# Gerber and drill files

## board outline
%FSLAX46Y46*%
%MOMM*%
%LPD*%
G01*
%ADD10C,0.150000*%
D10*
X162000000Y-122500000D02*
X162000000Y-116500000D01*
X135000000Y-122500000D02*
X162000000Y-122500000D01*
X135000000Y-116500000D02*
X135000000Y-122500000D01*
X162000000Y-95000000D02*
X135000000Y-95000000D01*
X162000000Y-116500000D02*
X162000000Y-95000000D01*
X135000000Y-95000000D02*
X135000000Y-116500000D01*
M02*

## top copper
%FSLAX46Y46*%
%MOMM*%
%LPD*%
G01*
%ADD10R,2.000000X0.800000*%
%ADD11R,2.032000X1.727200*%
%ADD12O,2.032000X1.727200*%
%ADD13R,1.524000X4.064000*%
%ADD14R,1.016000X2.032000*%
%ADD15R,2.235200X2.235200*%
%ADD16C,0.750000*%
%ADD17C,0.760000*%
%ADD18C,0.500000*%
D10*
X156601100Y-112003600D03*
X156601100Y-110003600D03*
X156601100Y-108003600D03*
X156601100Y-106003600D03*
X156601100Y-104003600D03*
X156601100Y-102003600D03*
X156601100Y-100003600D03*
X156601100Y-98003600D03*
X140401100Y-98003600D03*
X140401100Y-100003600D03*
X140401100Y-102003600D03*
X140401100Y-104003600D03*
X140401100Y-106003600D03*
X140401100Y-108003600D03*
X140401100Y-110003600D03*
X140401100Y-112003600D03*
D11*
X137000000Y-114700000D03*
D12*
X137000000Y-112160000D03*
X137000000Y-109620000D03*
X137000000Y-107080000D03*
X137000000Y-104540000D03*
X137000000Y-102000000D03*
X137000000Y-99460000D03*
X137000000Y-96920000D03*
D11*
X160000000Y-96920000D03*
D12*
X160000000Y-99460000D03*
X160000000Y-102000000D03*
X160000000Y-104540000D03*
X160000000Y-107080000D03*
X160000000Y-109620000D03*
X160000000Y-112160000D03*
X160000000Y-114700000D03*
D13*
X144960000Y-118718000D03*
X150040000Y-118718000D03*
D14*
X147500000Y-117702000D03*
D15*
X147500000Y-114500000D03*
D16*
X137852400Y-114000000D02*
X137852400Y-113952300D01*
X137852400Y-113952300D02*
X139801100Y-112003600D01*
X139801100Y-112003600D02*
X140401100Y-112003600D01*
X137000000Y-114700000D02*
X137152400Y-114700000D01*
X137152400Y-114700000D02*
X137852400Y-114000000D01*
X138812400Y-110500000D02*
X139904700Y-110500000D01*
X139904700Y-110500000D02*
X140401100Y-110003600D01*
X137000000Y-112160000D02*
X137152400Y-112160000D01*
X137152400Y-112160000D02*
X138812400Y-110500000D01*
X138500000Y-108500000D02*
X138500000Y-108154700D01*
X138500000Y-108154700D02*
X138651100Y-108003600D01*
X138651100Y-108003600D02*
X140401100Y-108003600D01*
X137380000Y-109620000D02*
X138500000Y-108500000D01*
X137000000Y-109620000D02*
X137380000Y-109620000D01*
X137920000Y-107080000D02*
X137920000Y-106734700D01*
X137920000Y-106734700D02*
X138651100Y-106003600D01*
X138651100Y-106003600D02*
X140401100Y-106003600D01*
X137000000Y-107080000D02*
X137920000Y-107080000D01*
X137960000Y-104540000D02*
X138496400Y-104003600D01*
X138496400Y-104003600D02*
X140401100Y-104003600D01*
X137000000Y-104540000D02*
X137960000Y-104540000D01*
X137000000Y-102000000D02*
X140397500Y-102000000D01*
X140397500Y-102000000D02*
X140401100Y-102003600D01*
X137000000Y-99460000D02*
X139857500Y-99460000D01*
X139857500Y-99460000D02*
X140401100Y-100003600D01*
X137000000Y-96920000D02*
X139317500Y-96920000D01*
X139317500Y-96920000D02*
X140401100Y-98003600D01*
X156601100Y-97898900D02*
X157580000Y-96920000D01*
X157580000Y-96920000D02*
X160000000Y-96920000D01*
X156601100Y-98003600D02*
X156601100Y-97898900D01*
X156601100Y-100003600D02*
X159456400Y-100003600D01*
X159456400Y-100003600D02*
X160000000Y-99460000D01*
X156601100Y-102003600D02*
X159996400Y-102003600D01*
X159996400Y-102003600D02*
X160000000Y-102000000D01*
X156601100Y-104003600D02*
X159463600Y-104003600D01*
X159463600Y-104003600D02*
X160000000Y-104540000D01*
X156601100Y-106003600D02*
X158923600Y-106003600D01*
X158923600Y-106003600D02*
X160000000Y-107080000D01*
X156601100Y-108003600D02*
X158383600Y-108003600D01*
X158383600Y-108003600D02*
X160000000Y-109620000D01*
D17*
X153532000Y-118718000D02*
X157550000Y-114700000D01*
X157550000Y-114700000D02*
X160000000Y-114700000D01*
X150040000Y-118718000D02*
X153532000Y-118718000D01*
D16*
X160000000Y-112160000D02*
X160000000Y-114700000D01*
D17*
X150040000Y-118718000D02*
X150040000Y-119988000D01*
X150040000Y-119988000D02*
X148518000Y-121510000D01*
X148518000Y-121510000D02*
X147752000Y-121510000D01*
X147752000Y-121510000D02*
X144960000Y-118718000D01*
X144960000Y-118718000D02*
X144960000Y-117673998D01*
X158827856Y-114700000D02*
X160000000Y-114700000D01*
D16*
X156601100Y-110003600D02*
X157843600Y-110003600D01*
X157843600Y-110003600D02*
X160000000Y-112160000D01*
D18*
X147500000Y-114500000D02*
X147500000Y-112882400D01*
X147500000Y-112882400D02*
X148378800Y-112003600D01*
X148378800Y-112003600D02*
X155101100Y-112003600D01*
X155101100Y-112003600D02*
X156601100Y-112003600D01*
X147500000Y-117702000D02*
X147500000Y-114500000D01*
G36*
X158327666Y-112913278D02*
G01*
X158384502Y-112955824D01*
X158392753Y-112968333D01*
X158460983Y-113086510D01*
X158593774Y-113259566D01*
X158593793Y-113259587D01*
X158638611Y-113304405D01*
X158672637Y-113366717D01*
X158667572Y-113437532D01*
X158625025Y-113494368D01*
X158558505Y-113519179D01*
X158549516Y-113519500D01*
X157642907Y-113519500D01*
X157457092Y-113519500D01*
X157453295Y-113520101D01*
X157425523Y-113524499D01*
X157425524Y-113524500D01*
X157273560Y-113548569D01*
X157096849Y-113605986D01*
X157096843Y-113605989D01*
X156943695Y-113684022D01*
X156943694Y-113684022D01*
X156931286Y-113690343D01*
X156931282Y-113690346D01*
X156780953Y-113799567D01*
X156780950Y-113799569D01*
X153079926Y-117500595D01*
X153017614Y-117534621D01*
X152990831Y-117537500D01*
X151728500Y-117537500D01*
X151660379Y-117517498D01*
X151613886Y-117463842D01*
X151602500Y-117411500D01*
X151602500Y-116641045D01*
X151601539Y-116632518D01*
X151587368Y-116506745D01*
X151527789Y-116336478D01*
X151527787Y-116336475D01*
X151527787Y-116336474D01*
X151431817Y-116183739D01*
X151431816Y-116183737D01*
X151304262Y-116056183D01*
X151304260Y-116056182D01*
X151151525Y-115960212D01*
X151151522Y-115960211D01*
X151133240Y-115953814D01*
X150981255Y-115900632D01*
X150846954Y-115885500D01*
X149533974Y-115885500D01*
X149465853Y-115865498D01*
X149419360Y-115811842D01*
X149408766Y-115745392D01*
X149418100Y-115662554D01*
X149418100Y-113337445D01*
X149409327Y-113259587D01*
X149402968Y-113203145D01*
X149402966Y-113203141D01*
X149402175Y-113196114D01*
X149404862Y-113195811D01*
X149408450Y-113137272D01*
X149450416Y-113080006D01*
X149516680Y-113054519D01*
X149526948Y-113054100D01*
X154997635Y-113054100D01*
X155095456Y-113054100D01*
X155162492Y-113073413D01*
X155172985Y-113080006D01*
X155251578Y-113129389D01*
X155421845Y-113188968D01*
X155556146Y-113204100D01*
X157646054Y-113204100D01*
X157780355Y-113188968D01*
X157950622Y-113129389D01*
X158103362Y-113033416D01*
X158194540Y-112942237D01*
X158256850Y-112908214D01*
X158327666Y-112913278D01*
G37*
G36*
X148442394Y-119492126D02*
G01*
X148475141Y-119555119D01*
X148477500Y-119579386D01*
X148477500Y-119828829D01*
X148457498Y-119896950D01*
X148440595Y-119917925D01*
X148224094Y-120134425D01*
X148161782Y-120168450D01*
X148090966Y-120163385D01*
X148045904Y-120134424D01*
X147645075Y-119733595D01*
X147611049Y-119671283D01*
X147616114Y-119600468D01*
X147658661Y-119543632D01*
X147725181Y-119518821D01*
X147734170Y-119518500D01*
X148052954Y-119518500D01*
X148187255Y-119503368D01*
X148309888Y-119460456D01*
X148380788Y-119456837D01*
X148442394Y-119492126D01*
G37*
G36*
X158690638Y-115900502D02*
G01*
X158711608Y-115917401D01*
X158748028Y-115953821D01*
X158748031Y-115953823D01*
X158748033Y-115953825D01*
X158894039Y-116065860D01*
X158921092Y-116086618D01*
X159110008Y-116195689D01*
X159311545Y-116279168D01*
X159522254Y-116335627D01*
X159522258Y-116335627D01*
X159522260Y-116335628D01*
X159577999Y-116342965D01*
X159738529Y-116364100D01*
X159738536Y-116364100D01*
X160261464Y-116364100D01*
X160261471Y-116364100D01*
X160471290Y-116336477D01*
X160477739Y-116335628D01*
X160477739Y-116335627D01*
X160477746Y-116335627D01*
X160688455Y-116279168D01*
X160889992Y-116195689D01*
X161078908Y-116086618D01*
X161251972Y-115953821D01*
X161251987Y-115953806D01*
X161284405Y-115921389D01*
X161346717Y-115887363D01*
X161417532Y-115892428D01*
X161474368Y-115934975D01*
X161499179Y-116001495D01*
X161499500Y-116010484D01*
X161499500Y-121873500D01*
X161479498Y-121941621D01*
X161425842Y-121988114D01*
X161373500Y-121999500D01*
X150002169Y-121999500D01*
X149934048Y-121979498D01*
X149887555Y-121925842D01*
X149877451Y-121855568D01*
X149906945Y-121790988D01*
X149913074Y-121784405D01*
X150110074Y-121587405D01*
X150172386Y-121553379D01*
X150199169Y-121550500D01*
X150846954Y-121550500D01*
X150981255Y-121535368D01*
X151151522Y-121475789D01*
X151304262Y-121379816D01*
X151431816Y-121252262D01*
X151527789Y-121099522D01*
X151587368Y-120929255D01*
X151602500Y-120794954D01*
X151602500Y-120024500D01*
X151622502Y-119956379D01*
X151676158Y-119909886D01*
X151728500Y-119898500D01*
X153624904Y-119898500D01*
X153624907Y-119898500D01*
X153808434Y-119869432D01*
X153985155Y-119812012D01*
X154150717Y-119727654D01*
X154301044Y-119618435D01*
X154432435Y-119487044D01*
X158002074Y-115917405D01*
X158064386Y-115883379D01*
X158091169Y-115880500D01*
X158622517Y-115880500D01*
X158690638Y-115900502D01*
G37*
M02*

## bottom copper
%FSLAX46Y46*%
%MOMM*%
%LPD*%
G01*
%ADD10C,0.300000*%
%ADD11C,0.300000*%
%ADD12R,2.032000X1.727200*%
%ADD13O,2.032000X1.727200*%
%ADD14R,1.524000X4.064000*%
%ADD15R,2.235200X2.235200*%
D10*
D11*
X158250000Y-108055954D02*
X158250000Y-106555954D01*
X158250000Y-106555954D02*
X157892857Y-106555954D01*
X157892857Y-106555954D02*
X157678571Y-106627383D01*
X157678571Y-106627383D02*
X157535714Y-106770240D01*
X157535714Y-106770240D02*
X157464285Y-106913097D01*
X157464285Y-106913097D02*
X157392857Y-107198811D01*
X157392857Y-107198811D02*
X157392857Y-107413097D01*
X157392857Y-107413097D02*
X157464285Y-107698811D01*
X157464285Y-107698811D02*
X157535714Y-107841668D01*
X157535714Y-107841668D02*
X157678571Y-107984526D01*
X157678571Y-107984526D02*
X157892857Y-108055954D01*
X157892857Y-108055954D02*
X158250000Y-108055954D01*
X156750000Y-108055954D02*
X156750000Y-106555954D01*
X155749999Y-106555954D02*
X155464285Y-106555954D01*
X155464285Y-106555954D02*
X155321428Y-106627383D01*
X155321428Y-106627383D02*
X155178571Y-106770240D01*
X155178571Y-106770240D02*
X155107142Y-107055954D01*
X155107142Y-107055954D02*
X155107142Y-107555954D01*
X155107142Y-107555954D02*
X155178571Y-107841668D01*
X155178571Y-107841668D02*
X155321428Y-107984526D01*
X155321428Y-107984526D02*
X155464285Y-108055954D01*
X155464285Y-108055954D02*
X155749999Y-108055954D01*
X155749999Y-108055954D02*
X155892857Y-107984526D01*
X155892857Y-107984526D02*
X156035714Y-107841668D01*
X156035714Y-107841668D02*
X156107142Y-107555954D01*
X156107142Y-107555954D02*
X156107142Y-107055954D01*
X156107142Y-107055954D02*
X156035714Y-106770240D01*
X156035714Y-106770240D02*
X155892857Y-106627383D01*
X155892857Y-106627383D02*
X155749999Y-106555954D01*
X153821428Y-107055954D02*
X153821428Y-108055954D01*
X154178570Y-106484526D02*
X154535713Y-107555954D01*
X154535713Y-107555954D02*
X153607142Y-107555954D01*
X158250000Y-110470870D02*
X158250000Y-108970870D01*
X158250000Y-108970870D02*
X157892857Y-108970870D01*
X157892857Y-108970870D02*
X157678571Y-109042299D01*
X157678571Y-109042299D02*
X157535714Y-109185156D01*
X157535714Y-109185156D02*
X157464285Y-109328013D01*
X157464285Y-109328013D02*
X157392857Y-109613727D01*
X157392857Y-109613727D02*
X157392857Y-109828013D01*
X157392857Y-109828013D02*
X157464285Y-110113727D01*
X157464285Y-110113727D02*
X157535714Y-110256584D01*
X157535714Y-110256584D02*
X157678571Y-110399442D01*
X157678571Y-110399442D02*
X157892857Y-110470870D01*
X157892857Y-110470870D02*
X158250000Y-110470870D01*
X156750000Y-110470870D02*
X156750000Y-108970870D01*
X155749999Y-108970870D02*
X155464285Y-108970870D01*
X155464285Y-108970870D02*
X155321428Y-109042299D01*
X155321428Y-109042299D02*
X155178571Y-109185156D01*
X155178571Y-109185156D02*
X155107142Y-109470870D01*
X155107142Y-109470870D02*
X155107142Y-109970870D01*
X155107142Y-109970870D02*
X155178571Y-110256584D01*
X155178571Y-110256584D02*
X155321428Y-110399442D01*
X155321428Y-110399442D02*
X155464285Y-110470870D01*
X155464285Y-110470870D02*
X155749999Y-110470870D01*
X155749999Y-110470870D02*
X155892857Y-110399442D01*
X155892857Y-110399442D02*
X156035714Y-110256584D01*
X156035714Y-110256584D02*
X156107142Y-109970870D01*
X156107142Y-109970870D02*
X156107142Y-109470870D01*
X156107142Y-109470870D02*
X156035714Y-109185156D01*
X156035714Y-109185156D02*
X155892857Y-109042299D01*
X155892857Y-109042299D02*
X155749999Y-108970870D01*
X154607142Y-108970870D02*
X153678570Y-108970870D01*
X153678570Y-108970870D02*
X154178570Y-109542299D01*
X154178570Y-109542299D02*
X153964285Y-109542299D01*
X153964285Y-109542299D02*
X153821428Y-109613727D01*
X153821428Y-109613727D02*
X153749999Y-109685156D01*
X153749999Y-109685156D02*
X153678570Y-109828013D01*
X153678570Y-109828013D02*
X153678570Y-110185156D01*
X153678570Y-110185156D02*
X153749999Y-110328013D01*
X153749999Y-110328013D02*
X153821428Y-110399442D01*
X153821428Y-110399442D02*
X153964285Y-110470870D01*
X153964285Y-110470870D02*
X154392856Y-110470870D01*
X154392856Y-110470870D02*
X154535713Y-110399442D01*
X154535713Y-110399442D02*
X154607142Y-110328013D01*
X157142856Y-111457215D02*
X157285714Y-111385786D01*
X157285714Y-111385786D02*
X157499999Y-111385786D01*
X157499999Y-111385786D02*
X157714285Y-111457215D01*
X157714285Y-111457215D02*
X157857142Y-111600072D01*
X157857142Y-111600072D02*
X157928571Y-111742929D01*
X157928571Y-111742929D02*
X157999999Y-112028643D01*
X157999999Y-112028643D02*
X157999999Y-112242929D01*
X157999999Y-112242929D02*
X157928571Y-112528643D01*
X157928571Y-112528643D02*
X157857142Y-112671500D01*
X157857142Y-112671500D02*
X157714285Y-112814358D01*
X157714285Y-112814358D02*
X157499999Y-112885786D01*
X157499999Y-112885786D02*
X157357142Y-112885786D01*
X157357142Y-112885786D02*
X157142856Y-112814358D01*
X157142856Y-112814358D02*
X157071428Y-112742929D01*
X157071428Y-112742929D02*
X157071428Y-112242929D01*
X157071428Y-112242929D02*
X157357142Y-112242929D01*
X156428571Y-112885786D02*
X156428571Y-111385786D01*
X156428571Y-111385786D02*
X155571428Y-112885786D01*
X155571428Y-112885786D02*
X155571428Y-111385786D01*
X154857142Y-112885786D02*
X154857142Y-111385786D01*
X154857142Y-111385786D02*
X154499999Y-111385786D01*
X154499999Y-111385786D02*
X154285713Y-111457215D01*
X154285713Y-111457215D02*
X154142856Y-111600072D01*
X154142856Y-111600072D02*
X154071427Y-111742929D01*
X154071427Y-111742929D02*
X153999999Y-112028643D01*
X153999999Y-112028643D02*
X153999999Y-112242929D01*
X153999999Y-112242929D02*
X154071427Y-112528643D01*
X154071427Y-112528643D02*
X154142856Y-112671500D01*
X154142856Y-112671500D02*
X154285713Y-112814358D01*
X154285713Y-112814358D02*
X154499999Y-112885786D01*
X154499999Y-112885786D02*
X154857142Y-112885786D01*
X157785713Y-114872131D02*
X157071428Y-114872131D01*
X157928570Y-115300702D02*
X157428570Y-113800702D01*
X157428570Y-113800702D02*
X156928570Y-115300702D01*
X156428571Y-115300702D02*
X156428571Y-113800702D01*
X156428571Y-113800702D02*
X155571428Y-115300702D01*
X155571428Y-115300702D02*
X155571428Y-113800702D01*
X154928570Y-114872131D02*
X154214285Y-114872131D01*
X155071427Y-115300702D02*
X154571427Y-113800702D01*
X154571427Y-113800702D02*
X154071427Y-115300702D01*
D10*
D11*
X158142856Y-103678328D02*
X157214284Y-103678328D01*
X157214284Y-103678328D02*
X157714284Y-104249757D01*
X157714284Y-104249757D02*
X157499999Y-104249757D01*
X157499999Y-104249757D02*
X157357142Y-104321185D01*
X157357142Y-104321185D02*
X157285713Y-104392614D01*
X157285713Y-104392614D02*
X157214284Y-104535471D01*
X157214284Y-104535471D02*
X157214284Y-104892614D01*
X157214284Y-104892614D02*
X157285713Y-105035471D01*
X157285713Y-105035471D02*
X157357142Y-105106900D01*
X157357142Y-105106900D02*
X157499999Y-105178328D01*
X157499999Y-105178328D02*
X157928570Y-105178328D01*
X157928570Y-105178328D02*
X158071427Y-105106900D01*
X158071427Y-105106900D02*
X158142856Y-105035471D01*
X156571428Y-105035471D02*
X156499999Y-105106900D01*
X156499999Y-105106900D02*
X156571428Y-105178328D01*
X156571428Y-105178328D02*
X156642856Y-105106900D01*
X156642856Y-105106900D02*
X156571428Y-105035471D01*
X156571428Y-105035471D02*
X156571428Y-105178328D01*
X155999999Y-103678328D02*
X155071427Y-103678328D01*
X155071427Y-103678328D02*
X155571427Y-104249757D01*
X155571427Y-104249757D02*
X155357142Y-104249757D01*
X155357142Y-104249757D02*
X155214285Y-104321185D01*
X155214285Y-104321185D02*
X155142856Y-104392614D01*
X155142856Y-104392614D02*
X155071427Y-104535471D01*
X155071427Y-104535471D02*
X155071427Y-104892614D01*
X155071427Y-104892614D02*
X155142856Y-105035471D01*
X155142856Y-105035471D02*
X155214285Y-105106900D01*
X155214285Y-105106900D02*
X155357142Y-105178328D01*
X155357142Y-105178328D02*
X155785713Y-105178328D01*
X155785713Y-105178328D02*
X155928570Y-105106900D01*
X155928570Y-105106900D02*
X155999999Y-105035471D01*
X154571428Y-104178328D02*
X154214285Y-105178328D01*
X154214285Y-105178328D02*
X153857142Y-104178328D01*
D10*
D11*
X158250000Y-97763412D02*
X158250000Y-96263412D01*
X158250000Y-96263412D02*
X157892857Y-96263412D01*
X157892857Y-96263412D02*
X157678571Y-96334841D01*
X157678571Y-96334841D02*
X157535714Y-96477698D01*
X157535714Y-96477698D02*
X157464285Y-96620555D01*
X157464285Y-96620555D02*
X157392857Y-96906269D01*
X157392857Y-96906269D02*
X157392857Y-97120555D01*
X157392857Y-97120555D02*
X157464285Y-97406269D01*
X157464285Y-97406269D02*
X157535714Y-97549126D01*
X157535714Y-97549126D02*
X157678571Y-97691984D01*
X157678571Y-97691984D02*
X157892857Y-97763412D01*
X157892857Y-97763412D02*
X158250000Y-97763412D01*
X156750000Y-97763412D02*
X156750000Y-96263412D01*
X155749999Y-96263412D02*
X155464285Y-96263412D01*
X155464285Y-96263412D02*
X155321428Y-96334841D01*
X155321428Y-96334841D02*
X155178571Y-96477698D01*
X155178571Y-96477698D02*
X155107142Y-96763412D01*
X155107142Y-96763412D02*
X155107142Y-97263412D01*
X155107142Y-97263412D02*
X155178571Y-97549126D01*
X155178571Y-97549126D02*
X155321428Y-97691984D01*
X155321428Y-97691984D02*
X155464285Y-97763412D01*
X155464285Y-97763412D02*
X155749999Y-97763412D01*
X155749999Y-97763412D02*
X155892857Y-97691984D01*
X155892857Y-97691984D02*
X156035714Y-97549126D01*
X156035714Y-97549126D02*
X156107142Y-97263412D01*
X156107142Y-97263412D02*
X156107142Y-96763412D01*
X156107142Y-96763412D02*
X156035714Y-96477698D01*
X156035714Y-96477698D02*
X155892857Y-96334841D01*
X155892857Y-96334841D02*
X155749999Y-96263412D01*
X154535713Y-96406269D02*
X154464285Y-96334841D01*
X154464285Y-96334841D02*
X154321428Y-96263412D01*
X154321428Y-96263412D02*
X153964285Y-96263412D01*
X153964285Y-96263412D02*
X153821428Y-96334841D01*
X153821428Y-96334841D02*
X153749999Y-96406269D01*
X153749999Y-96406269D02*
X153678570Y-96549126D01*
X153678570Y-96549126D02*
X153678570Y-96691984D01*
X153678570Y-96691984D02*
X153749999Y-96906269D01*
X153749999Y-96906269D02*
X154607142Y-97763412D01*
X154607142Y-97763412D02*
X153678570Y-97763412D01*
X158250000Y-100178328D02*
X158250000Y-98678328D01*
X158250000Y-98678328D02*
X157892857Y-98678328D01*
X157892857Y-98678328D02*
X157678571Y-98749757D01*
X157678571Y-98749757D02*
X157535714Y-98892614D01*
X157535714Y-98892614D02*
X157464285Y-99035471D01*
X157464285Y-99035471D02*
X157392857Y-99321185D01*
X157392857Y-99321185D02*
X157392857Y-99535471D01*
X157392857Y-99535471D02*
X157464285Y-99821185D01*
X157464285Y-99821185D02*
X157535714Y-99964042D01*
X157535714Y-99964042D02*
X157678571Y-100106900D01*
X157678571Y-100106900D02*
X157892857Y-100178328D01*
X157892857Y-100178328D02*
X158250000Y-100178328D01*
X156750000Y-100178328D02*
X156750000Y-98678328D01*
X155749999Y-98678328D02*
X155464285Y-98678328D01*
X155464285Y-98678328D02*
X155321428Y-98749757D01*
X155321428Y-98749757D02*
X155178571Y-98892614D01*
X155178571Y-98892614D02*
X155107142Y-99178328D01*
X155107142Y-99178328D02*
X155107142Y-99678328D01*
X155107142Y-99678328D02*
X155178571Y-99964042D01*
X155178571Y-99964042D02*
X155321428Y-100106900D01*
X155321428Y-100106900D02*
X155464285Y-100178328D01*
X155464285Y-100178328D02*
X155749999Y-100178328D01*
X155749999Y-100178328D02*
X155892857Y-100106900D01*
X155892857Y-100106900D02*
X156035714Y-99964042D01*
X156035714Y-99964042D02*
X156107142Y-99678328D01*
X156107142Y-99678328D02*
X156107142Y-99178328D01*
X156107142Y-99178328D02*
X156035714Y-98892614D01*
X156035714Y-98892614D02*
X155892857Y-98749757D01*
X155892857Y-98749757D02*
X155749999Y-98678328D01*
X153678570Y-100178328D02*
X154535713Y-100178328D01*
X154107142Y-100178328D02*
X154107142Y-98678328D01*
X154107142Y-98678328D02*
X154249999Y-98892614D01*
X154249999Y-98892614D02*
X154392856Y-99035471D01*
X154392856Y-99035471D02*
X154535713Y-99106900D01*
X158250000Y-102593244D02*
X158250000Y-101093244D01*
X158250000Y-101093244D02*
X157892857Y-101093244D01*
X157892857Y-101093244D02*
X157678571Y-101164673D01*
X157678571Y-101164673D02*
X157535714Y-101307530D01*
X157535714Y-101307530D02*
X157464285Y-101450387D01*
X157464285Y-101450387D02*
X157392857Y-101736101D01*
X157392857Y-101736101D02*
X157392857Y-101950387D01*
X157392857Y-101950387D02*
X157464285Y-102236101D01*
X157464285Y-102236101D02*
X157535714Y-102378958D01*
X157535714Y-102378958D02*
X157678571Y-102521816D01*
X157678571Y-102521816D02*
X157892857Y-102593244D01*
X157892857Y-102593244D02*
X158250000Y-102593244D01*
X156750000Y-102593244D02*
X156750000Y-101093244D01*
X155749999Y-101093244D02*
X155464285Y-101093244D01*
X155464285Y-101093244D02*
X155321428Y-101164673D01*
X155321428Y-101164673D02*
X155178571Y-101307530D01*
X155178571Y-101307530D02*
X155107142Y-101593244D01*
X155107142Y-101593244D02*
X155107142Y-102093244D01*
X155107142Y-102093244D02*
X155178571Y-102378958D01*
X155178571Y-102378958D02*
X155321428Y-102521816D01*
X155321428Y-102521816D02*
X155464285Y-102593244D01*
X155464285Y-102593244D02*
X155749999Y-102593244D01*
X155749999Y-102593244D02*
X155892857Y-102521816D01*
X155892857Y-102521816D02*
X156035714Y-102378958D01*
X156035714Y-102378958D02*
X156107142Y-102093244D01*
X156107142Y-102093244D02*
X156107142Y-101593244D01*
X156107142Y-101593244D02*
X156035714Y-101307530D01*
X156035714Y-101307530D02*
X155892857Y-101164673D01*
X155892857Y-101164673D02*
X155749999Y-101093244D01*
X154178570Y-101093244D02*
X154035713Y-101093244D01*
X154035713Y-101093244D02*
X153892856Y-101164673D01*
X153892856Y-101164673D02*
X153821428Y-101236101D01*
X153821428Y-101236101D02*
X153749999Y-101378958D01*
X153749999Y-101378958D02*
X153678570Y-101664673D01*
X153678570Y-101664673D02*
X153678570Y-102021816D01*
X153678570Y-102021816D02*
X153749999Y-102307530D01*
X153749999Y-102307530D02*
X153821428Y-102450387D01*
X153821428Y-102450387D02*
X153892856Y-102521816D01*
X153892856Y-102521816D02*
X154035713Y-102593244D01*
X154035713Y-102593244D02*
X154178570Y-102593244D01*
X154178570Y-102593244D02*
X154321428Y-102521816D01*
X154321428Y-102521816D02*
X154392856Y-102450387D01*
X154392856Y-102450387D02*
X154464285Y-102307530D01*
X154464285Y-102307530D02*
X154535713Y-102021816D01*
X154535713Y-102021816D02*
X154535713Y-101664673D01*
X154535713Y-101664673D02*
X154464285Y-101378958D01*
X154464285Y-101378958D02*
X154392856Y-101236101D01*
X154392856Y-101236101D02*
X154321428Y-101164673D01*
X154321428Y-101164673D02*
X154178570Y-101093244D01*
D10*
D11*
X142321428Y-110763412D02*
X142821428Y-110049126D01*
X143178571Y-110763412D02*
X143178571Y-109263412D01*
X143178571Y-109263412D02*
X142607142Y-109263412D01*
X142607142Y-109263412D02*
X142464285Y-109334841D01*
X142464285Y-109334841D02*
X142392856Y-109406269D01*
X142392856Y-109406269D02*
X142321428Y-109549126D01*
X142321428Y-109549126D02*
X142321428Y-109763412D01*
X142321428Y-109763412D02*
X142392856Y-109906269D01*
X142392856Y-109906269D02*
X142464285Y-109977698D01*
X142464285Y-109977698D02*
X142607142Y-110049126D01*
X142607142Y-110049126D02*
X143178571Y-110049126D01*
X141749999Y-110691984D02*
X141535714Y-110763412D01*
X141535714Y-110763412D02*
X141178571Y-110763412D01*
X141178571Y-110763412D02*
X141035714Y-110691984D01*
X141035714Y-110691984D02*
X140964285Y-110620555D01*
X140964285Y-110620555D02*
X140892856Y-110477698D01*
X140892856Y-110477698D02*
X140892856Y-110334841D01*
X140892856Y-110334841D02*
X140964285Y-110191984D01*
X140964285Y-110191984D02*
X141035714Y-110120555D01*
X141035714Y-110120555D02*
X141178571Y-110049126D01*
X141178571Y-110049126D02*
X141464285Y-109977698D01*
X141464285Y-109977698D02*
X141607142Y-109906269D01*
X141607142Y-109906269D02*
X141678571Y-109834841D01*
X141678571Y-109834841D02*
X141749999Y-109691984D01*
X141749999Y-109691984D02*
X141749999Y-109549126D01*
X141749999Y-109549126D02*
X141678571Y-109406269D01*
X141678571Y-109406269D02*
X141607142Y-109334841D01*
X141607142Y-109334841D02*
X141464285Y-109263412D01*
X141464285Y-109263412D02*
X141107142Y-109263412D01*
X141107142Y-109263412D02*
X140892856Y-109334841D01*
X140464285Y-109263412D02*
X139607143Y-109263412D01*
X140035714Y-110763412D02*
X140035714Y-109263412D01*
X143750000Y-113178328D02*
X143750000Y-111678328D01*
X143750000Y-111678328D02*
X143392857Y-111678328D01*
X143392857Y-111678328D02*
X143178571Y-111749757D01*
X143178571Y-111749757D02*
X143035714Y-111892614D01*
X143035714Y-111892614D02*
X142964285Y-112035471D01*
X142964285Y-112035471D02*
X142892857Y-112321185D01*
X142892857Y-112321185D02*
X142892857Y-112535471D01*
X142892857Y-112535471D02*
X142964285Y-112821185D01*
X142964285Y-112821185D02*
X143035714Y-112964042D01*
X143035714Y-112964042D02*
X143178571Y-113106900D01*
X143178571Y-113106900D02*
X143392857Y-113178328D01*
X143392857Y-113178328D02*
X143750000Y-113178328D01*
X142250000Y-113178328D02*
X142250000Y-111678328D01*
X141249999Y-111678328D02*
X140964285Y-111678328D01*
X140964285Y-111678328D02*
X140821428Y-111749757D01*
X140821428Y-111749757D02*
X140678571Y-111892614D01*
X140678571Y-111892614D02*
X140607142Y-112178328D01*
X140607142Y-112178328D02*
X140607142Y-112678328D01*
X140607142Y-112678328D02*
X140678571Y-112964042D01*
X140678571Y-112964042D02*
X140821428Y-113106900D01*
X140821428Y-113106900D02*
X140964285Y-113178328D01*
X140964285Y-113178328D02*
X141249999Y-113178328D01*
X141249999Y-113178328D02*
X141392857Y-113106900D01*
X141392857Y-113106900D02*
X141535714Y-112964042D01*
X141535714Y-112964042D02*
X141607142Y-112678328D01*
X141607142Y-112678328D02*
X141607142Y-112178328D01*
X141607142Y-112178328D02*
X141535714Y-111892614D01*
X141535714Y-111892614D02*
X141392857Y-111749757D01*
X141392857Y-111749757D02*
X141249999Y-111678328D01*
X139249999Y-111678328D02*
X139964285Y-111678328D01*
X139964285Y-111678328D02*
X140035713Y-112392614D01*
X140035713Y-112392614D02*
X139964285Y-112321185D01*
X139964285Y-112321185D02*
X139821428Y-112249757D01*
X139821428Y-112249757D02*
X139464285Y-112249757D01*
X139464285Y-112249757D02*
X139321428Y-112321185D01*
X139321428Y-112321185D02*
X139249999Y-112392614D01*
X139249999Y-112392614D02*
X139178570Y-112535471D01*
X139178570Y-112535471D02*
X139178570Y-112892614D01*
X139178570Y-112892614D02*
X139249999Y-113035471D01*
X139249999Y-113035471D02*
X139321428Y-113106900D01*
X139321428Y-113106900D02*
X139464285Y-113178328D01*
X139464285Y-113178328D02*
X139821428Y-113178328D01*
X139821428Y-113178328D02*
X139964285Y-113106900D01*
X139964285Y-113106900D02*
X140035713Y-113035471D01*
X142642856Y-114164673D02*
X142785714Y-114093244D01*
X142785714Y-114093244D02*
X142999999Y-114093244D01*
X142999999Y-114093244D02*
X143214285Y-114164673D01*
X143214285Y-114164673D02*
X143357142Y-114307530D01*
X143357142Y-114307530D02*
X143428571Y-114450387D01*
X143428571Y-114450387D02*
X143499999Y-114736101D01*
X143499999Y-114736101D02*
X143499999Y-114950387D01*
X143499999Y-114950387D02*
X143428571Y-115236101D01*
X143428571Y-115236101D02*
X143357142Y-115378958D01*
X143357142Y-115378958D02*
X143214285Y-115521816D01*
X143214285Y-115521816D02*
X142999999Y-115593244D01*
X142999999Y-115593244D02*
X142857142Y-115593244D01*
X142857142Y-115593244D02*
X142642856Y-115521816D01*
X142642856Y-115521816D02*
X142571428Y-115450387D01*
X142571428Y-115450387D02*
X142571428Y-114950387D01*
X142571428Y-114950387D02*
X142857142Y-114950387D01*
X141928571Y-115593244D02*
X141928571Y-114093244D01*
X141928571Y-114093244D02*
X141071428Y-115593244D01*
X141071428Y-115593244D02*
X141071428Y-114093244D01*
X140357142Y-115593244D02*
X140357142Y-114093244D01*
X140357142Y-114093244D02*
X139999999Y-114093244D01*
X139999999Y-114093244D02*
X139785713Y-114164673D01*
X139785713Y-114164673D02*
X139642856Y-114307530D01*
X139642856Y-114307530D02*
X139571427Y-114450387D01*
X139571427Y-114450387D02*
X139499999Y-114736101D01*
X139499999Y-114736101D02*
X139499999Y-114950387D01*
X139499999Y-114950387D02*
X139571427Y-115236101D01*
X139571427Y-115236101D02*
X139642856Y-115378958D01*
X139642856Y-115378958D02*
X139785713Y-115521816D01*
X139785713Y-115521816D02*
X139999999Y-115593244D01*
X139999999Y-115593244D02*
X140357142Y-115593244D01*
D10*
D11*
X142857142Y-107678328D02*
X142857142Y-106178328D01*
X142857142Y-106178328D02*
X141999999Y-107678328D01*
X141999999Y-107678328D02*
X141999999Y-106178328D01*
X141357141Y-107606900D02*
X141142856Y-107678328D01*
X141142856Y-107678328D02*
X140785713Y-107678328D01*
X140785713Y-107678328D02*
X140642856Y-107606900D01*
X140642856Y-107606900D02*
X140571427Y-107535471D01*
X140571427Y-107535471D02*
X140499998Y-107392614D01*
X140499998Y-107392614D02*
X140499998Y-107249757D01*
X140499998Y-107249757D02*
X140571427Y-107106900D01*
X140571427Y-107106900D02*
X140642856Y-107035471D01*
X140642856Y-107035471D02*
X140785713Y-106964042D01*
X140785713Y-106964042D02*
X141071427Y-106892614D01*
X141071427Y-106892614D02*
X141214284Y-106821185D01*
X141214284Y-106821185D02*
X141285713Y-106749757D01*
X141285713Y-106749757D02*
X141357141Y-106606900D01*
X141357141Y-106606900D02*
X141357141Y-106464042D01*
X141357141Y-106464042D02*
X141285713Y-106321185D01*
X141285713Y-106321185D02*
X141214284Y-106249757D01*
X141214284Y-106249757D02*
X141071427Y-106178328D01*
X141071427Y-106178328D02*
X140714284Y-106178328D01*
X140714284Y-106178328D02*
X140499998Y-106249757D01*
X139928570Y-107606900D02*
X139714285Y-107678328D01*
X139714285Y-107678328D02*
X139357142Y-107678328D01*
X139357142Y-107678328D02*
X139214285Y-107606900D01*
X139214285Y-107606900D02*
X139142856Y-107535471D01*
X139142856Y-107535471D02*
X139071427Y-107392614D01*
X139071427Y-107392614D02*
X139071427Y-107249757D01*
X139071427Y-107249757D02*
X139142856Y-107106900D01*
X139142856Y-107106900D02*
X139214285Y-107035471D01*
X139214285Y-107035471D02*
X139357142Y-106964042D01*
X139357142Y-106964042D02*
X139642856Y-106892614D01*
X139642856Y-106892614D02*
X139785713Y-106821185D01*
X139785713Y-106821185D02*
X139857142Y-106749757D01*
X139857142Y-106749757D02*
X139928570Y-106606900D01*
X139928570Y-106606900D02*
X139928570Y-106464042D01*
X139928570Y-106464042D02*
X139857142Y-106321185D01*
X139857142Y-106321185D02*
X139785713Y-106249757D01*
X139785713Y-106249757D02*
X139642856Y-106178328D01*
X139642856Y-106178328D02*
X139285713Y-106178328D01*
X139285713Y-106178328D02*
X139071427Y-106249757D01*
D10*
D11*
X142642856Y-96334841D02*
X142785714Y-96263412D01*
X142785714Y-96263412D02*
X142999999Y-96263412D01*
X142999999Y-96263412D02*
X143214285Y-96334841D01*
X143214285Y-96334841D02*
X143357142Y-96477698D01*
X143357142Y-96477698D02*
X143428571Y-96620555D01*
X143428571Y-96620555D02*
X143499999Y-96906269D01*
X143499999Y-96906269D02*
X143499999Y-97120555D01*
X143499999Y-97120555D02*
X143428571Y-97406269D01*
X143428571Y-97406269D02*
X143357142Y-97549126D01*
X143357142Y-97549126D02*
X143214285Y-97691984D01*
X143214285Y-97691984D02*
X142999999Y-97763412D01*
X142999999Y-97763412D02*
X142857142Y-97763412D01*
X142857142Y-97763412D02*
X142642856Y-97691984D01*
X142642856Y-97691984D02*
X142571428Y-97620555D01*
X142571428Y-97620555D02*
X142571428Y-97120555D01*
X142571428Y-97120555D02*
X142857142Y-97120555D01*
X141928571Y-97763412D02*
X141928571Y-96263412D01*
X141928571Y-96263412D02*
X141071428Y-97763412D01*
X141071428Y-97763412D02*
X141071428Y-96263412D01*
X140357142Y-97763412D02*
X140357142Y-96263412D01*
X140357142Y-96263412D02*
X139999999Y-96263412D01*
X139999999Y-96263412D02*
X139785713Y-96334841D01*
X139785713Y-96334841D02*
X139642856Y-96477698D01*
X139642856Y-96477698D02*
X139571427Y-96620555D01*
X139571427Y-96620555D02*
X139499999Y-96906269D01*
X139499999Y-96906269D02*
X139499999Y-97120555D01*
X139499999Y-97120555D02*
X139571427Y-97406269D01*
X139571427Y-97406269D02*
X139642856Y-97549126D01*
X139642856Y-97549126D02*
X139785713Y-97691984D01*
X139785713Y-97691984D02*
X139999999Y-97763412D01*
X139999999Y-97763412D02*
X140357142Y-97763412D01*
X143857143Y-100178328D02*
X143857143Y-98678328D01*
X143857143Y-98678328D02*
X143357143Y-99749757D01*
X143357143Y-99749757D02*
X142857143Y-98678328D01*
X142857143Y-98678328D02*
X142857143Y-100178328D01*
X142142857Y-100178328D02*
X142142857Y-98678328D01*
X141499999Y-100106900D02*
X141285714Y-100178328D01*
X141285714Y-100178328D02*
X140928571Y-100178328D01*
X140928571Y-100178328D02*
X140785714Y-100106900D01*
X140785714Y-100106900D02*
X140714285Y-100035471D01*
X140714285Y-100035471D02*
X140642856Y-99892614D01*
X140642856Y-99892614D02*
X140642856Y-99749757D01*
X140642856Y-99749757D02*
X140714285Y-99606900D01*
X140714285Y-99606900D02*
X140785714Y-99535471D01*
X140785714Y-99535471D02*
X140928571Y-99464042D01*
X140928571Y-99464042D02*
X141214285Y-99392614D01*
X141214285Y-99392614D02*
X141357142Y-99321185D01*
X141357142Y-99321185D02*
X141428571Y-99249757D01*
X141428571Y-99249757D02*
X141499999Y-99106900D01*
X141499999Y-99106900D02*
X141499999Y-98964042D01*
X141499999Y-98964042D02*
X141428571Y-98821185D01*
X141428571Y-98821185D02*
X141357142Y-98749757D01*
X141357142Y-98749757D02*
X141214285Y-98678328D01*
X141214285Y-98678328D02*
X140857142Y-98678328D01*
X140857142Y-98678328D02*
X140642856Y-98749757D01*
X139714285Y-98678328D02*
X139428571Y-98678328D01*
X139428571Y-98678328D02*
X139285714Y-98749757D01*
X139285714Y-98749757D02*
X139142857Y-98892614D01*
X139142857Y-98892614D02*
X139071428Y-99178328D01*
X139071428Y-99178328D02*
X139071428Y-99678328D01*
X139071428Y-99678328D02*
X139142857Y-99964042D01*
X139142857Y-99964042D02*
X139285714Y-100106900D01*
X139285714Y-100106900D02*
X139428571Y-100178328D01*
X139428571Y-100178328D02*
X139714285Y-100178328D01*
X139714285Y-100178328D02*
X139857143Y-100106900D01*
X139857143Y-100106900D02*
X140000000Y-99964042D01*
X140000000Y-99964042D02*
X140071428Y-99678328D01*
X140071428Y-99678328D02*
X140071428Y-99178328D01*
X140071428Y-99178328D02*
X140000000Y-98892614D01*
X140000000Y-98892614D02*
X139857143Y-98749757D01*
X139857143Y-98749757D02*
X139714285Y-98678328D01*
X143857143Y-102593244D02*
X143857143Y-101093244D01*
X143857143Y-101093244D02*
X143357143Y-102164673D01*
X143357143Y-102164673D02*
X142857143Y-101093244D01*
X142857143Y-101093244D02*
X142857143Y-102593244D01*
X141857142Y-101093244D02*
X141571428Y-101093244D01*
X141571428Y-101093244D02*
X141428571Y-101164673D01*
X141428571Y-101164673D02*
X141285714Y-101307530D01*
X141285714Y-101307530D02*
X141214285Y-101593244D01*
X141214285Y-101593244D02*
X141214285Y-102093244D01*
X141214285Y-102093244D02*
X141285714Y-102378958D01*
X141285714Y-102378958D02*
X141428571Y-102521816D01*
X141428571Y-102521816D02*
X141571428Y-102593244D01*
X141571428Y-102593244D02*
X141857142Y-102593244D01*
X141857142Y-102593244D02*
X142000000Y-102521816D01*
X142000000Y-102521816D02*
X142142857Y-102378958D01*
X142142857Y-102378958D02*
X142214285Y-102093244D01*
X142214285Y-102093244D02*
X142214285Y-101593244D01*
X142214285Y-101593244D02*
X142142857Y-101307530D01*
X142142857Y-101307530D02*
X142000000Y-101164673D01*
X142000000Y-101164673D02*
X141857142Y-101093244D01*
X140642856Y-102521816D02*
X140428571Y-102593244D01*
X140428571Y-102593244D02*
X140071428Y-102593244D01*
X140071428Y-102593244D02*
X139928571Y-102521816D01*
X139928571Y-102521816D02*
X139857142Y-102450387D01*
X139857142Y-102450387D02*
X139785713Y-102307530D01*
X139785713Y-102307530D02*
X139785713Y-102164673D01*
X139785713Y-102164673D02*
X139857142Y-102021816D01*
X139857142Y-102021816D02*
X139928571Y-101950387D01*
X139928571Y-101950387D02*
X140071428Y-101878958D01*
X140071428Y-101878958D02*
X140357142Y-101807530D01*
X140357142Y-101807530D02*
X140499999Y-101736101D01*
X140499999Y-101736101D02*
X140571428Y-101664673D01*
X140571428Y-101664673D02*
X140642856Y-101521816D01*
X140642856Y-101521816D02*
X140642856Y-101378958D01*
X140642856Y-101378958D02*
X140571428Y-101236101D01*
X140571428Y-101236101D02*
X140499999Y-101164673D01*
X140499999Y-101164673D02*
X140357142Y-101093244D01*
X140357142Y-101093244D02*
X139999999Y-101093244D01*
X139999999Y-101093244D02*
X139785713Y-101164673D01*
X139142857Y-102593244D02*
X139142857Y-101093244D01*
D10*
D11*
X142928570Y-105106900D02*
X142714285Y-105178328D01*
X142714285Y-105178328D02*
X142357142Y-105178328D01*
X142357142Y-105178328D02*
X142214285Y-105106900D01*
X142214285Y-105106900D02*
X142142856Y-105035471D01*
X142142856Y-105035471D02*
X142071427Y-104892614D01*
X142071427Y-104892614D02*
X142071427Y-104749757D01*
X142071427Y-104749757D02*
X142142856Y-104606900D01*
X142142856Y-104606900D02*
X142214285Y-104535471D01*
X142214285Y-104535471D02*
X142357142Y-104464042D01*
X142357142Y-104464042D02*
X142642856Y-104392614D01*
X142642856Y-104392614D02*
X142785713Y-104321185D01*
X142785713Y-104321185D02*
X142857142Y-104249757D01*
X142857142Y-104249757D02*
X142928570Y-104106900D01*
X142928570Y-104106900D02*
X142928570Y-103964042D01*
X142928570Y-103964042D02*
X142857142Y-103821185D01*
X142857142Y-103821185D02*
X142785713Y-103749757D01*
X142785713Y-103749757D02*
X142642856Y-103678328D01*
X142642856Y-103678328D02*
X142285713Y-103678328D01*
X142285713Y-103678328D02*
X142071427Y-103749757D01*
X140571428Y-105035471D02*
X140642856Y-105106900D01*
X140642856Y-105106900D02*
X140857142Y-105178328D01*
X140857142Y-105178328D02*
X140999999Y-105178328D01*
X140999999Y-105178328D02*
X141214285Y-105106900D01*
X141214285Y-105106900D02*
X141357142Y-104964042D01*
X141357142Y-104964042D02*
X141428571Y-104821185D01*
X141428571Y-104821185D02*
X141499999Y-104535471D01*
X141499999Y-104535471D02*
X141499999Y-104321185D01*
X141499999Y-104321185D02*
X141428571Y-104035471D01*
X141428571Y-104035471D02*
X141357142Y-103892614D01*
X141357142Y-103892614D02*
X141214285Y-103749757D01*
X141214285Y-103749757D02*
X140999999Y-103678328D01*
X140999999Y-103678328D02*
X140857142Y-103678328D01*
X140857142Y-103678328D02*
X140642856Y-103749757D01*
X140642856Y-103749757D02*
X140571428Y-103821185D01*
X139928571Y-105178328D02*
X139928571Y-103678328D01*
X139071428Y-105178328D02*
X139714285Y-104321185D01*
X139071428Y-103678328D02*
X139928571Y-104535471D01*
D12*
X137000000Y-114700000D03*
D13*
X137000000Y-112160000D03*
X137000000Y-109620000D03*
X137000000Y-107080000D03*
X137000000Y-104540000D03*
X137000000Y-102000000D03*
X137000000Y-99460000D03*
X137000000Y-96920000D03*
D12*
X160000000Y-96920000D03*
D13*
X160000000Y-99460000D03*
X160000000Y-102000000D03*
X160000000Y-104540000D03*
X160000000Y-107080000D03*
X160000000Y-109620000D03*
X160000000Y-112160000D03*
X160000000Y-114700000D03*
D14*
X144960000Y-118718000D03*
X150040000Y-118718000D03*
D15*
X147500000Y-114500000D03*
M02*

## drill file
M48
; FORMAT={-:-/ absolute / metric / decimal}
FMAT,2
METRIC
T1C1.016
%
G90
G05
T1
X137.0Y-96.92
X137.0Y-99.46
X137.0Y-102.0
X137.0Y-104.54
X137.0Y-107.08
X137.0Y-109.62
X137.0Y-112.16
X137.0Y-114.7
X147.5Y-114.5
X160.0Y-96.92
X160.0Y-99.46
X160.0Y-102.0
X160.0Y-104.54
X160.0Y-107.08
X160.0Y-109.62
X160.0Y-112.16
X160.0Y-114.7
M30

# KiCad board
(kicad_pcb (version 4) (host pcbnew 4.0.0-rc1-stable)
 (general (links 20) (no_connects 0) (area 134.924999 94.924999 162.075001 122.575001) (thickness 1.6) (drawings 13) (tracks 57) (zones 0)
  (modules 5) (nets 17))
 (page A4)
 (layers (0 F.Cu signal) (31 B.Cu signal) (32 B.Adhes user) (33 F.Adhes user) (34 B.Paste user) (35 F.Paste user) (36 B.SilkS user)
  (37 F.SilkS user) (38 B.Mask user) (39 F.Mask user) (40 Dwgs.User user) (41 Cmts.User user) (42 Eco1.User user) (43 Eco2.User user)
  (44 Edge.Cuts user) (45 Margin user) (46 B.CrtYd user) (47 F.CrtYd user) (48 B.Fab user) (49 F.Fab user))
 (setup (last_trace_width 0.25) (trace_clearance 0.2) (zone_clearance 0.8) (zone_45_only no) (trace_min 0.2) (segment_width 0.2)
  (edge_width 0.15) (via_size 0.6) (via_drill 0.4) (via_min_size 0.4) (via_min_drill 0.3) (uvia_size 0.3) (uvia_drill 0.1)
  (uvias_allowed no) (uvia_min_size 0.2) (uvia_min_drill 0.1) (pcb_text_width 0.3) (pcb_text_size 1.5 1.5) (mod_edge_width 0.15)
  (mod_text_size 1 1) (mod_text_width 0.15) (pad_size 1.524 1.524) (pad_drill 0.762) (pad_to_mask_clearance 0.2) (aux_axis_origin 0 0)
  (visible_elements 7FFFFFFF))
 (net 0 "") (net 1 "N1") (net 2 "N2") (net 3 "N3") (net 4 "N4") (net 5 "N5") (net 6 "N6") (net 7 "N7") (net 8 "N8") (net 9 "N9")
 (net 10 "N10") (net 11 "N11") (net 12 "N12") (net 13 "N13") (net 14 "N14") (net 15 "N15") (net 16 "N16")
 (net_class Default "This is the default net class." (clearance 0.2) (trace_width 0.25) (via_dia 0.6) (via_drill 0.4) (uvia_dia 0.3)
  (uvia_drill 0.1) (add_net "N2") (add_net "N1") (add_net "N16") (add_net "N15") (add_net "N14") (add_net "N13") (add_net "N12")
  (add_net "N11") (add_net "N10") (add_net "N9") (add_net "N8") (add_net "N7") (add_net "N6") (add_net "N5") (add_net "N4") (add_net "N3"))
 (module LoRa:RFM (layer F.Cu) (at 148.5011 105.0036)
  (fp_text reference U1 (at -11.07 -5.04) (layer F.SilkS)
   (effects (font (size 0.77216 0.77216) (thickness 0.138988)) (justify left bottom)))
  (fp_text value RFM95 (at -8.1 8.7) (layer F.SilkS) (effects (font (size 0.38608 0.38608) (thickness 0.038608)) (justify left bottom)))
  (pad 16 smd rect (at 8.1 7 180) (size 2 0.8) (layers F.Cu F.Paste F.Mask) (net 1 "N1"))
  (pad 15 smd rect (at 8.1 5 180) (size 2 0.8) (layers F.Cu F.Paste F.Mask) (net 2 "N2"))
  (pad 14 smd rect (at 8.1 3 180) (size 2 0.8) (layers F.Cu F.Paste F.Mask) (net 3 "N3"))
  (pad 13 smd rect (at 8.1 1 180) (size 2 0.8) (layers F.Cu F.Paste F.Mask) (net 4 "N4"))
  (pad 12 smd rect (at 8.1 -1 180) (size 2 0.8) (layers F.Cu F.Paste F.Mask) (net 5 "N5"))
  (pad 11 smd rect (at 8.1 -3 180) (size 2 0.8) (layers F.Cu F.Paste F.Mask) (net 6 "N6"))
  (pad 10 smd rect (at 8.1 -5 180) (size 2 0.8) (layers F.Cu F.Paste F.Mask) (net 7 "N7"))
  (pad 9 smd rect (at 8.1 -7 180) (size 2 0.8) (layers F.Cu F.Paste F.Mask) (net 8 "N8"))
  (pad 1 smd rect (at -8.1 -7) (size 2 0.8) (layers F.Cu F.Paste F.Mask) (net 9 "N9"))
  (pad 2 smd rect (at -8.1 -5) (size 2 0.8) (layers F.Cu F.Paste F.Mask) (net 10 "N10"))
  (pad 3 smd rect (at -8.1 -3) (size 2 0.8) (layers F.Cu F.Paste F.Mask) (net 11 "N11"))
  (pad 4 smd rect (at -8.1 -1) (size 2 0.8) (layers F.Cu F.Paste F.Mask) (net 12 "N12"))
  (pad 5 smd rect (at -8.1 1) (size 2 0.8) (layers F.Cu F.Paste F.Mask) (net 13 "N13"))
  (pad 6 smd rect (at -8.1 3) (size 2 0.8) (layers F.Cu F.Paste F.Mask) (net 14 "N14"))
  (pad 7 smd rect (at -8.1 5) (size 2 0.8) (layers F.Cu F.Paste F.Mask) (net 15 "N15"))
  (pad 8 smd rect (at -8.1 7 180) (size 2 0.8) (layers F.Cu F.Paste F.Mask) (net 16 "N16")))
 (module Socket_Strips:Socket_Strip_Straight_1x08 (layer F.Cu) (at 137 114.7 90)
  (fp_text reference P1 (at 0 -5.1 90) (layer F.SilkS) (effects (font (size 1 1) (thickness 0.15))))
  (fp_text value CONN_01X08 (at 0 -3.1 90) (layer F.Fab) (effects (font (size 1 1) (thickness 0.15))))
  (pad 1 thru_hole rect (at 0 0 90) (size 1.7272 2.032) (drill 1.016) (layers *.Cu *.Mask F.SilkS) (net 16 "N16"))
  (pad 2 thru_hole oval (at 2.54 0 90) (size 1.7272 2.032) (drill 1.016) (layers *.Cu *.Mask F.SilkS) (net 15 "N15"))
  (pad 3 thru_hole oval (at 5.08 0 90) (size 1.7272 2.032) (drill 1.016) (layers *.Cu *.Mask F.SilkS) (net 14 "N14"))
  (pad 4 thru_hole oval (at 7.62 0 90) (size 1.7272 2.032) (drill 1.016) (layers *.Cu *.Mask F.SilkS) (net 13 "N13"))
  (pad 5 thru_hole oval (at 10.16 0 90) (size 1.7272 2.032) (drill 1.016) (layers *.Cu *.Mask F.SilkS) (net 12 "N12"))
  (pad 6 thru_hole oval (at 12.7 0 90) (size 1.7272 2.032) (drill 1.016) (layers *.Cu *.Mask F.SilkS) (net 11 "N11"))
  (pad 7 thru_hole oval (at 15.24 0 90) (size 1.7272 2.032) (drill 1.016) (layers *.Cu *.Mask F.SilkS) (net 10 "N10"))
  (pad 8 thru_hole oval (at 17.78 0 90) (size 1.7272 2.032) (drill 1.016) (layers *.Cu *.Mask F.SilkS) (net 9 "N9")))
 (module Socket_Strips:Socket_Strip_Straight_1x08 (layer F.Cu) (at 160 96.92 270)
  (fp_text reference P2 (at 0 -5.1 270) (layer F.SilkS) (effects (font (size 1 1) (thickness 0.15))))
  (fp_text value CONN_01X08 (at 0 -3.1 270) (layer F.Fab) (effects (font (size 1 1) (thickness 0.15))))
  (pad 1 thru_hole rect (at 0 0 270) (size 1.7272 2.032) (drill 1.016) (layers *.Cu *.Mask F.SilkS) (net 8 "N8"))
  (pad 2 thru_hole oval (at 2.54 0 270) (size 1.7272 2.032) (drill 1.016) (layers *.Cu *.Mask F.SilkS) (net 7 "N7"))
  (pad 3 thru_hole oval (at 5.08 0 270) (size 1.7272 2.032) (drill 1.016) (layers *.Cu *.Mask F.SilkS) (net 6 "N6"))
  (pad 4 thru_hole oval (at 7.62 0 270) (size 1.7272 2.032) (drill 1.016) (layers *.Cu *.Mask F.SilkS) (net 5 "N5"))
  (pad 5 thru_hole oval (at 10.16 0 270) (size 1.7272 2.032) (drill 1.016) (layers *.Cu *.Mask F.SilkS) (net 4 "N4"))
  (pad 6 thru_hole oval (at 12.7 0 270) (size 1.7272 2.032) (drill 1.016) (layers *.Cu *.Mask F.SilkS) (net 3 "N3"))
  (pad 7 thru_hole oval (at 15.24 0 270) (size 1.7272 2.032) (drill 1.016) (layers *.Cu *.Mask F.SilkS) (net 2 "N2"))
  (pad 8 thru_hole oval (at 17.78 0 270) (size 1.7272 2.032) (drill 1.016) (layers *.Cu *.Mask F.SilkS) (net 2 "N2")))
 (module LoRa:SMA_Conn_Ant (layer F.Cu) (at 147.5 120.75 90)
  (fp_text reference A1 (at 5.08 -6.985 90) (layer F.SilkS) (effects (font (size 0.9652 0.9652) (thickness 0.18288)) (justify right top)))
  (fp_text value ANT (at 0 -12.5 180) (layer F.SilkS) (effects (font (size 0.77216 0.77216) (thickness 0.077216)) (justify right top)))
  (pad 1 smd rect (at 2.032 -2.54 180) (size 1.524 4.064) (layers F.Cu F.Paste F.Mask) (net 2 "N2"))
  (pad 3 smd rect (at 2.032 2.54 180) (size 1.524 4.064) (layers F.Cu F.Paste F.Mask) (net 2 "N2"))
  (pad 2 smd rect (at 3.048 0 180) (size 1.016 2.032) (layers F.Cu F.Paste F.Mask) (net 1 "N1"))
  (pad "" smd rect (at 2.032 -2.54 180) (size 1.524 4.064) (layers B.Cu B.Paste B.Mask))
  (pad "" smd rect (at 2.032 2.54 180) (size 1.524 4.064) (layers B.Cu B.Paste B.Mask)))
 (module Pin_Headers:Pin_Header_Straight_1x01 (layer F.Cu) (at 147.5 114.5)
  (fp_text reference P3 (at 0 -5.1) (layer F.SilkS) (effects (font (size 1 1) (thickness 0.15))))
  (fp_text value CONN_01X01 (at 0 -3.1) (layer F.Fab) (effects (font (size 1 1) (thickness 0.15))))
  (pad 1 thru_hole rect (at 0 0) (size 2.2352 2.2352) (drill 1.016) (layers *.Cu *.Mask F.SilkS) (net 1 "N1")))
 (gr_line (start 162 122.5) (end 162 116.5) (angle 90) (layer Edge.Cuts) (width 0.15))
 (gr_line (start 135 122.5) (end 162 122.5) (angle 90) (layer Edge.Cuts) (width 0.15))
 (gr_line (start 135 116.5) (end 135 122.5) (angle 90) (layer Edge.Cuts) (width 0.15))
 (gr_line (start 162 95) (end 135 95) (layer Edge.Cuts) (width 0.15))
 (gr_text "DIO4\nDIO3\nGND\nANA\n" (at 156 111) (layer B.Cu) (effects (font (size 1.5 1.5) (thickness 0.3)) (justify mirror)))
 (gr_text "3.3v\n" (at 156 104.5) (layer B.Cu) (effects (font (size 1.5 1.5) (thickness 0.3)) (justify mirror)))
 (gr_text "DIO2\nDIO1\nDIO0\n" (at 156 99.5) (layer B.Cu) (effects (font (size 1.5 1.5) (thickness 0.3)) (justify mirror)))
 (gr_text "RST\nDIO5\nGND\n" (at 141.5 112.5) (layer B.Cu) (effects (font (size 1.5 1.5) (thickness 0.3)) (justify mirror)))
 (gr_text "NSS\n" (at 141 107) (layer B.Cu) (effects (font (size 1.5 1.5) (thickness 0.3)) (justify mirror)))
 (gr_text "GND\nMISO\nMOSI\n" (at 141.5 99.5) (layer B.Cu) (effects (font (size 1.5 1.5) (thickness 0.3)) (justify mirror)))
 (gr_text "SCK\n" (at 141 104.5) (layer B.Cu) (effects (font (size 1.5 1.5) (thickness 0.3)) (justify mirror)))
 (gr_line (start 162 116.5) (end 162 95) (layer Edge.Cuts) (width 0.15))
 (gr_line (start 135 95) (end 135 116.5) (layer Edge.Cuts) (width 0.15))
 (segment (start 137.8524 114) (end 137.8524 113.9523) (width 0.75) (layer F.Cu) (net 16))
 (segment (start 137.8524 113.9523) (end 139.8011 112.0036) (width 0.75) (layer F.Cu) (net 16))
 (segment (start 139.8011 112.0036) (end 140.4011 112.0036) (width 0.75) (layer F.Cu) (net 16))
 (segment (start 137 114.7) (end 137.1524 114.7) (width 0.75) (layer F.Cu) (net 16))
 (segment (start 137.1524 114.7) (end 137.8524 114) (width 0.75) (layer F.Cu) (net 16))
 (segment (start 138.8124 110.5) (end 139.9047 110.5) (width 0.75) (layer F.Cu) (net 15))
 (segment (start 139.9047 110.5) (end 140.4011 110.0036) (width 0.75) (layer F.Cu) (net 15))
 (segment (start 137 112.16) (end 137.1524 112.16) (width 0.75) (layer F.Cu) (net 15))
 (segment (start 137.1524 112.16) (end 138.8124 110.5) (width 0.75) (layer F.Cu) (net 15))
 (segment (start 138.5 108.5) (end 138.5 108.1547) (width 0.75) (layer F.Cu) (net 14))
 (segment (start 138.5 108.1547) (end 138.6511 108.0036) (width 0.75) (layer F.Cu) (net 14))
 (segment (start 138.6511 108.0036) (end 140.4011 108.0036) (width 0.75) (layer F.Cu) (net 14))
 (segment (start 137.38 109.62) (end 138.5 108.5) (width 0.75) (layer F.Cu) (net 14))
 (segment (start 137 109.62) (end 137.38 109.62) (width 0.75) (layer F.Cu) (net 14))
 (segment (start 137.92 107.08) (end 137.92 106.7347) (width 0.75) (layer F.Cu) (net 13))
 (segment (start 137.92 106.7347) (end 138.6511 106.0036) (width 0.75) (layer F.Cu) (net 13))
 (segment (start 138.6511 106.0036) (end 140.4011 106.0036) (width 0.75) (layer F.Cu) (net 13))
 (segment (start 137 107.08) (end 137.92 107.08) (width 0.75) (layer F.Cu) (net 13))
 (segment (start 137.96 104.54) (end 138.4964 104.0036) (width 0.75) (layer F.Cu) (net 12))
 (segment (start 138.4964 104.0036) (end 140.4011 104.0036) (width 0.75) (layer F.Cu) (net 12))
 (segment (start 137 104.54) (end 137.96 104.54) (width 0.75) (layer F.Cu) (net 12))
 (segment (start 137 102) (end 140.3975 102) (width 0.75) (layer F.Cu) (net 11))
 (segment (start 140.3975 102) (end 140.4011 102.0036) (width 0.75) (layer F.Cu) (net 11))
 (segment (start 137 99.46) (end 139.8575 99.46) (width 0.75) (layer F.Cu) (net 10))
 (segment (start 139.8575 99.46) (end 140.4011 100.0036) (width 0.75) (layer F.Cu) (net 10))
 (segment (start 137 96.92) (end 139.3175 96.92) (width 0.75) (layer F.Cu) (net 9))
 (segment (start 139.3175 96.92) (end 140.4011 98.0036) (width 0.75) (layer F.Cu) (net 9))
 (segment (start 156.6011 97.8989) (end 157.58 96.92) (width 0.75) (layer F.Cu) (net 8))
 (segment (start 157.58 96.92) (end 160 96.92) (width 0.75) (layer F.Cu) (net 8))
 (segment (start 156.6011 98.0036) (end 156.6011 97.8989) (width 0.75) (layer F.Cu) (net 8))
 (segment (start 156.6011 100.0036) (end 159.4564 100.0036) (width 0.75) (layer F.Cu) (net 7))
 (segment (start 159.4564 100.0036) (end 160 99.46) (width 0.75) (layer F.Cu) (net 7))
 (segment (start 156.6011 102.0036) (end 159.9964 102.0036) (width 0.75) (layer F.Cu) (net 6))
 (segment (start 159.9964 102.0036) (end 160 102) (width 0.75) (layer F.Cu) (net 6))
 (segment (start 156.6011 104.0036) (end 159.4636 104.0036) (width 0.75) (layer F.Cu) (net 5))
 (segment (start 159.4636 104.0036) (end 160 104.54) (width 0.75) (layer F.Cu) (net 5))
 (segment (start 156.6011 106.0036) (end 158.9236 106.0036) (width 0.75) (layer F.Cu) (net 4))
 (segment (start 158.9236 106.0036) (end 160 107.08) (width 0.75) (layer F.Cu) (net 4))
 (segment (start 156.6011 108.0036) (end 158.3836 108.0036) (width 0.75) (layer F.Cu) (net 3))
 (segment (start 158.3836 108.0036) (end 160 109.62) (width 0.75) (layer F.Cu) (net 3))
 (segment (start 153.532 118.718) (end 157.55 114.7) (width 0.76) (layer F.Cu) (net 2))
 (segment (start 157.55 114.7) (end 160 114.7) (width 0.76) (layer F.Cu) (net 2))
 (segment (start 150.04 118.718) (end 153.532 118.718) (width 0.76) (layer F.Cu) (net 2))
 (segment (start 160 112.16) (end 160 114.7) (width 0.75) (layer F.Cu) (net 2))
 (segment (start 150.04 118.718) (end 150.04 119.988) (width 0.76) (layer F.Cu) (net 2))
 (segment (start 150.04 119.988) (end 148.518 121.51) (width 0.76) (layer F.Cu) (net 2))
 (segment (start 148.518 121.51) (end 147.752 121.51) (width 0.76) (layer F.Cu) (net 2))
 (segment (start 147.752 121.51) (end 144.96 118.718) (width 0.76) (layer F.Cu) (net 2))
 (segment (start 144.96 118.718) (end 144.96 117.673998) (width 0.76) (layer F.Cu) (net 2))
 (segment (start 158.827856 114.7) (end 160 114.7) (width 0.76) (layer F.Cu) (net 2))
 (segment (start 156.6011 110.0036) (end 157.8436 110.0036) (width 0.75) (layer F.Cu) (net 2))
 (segment (start 157.8436 110.0036) (end 160 112.16) (width 0.75) (layer F.Cu) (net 2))
 (segment (start 147.5 114.5) (end 147.5 112.8824) (width 0.5) (layer F.Cu) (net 1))
 (segment (start 147.5 112.8824) (end 148.3788 112.0036) (width 0.5) (layer F.Cu) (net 1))
 (segment (start 148.3788 112.0036) (end 155.1011 112.0036) (width 0.5) (layer F.Cu) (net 1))
 (segment (start 155.1011 112.0036) (end 156.6011 112.0036) (width 0.5) (layer F.Cu) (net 1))
 (segment (start 147.5 117.702) (end 147.5 114.5) (width 0.5) (layer F.Cu) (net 1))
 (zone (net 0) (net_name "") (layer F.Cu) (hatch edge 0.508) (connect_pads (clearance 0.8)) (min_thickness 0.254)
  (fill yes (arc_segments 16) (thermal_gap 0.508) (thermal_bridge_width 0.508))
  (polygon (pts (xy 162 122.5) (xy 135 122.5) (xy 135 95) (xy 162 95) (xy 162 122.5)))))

